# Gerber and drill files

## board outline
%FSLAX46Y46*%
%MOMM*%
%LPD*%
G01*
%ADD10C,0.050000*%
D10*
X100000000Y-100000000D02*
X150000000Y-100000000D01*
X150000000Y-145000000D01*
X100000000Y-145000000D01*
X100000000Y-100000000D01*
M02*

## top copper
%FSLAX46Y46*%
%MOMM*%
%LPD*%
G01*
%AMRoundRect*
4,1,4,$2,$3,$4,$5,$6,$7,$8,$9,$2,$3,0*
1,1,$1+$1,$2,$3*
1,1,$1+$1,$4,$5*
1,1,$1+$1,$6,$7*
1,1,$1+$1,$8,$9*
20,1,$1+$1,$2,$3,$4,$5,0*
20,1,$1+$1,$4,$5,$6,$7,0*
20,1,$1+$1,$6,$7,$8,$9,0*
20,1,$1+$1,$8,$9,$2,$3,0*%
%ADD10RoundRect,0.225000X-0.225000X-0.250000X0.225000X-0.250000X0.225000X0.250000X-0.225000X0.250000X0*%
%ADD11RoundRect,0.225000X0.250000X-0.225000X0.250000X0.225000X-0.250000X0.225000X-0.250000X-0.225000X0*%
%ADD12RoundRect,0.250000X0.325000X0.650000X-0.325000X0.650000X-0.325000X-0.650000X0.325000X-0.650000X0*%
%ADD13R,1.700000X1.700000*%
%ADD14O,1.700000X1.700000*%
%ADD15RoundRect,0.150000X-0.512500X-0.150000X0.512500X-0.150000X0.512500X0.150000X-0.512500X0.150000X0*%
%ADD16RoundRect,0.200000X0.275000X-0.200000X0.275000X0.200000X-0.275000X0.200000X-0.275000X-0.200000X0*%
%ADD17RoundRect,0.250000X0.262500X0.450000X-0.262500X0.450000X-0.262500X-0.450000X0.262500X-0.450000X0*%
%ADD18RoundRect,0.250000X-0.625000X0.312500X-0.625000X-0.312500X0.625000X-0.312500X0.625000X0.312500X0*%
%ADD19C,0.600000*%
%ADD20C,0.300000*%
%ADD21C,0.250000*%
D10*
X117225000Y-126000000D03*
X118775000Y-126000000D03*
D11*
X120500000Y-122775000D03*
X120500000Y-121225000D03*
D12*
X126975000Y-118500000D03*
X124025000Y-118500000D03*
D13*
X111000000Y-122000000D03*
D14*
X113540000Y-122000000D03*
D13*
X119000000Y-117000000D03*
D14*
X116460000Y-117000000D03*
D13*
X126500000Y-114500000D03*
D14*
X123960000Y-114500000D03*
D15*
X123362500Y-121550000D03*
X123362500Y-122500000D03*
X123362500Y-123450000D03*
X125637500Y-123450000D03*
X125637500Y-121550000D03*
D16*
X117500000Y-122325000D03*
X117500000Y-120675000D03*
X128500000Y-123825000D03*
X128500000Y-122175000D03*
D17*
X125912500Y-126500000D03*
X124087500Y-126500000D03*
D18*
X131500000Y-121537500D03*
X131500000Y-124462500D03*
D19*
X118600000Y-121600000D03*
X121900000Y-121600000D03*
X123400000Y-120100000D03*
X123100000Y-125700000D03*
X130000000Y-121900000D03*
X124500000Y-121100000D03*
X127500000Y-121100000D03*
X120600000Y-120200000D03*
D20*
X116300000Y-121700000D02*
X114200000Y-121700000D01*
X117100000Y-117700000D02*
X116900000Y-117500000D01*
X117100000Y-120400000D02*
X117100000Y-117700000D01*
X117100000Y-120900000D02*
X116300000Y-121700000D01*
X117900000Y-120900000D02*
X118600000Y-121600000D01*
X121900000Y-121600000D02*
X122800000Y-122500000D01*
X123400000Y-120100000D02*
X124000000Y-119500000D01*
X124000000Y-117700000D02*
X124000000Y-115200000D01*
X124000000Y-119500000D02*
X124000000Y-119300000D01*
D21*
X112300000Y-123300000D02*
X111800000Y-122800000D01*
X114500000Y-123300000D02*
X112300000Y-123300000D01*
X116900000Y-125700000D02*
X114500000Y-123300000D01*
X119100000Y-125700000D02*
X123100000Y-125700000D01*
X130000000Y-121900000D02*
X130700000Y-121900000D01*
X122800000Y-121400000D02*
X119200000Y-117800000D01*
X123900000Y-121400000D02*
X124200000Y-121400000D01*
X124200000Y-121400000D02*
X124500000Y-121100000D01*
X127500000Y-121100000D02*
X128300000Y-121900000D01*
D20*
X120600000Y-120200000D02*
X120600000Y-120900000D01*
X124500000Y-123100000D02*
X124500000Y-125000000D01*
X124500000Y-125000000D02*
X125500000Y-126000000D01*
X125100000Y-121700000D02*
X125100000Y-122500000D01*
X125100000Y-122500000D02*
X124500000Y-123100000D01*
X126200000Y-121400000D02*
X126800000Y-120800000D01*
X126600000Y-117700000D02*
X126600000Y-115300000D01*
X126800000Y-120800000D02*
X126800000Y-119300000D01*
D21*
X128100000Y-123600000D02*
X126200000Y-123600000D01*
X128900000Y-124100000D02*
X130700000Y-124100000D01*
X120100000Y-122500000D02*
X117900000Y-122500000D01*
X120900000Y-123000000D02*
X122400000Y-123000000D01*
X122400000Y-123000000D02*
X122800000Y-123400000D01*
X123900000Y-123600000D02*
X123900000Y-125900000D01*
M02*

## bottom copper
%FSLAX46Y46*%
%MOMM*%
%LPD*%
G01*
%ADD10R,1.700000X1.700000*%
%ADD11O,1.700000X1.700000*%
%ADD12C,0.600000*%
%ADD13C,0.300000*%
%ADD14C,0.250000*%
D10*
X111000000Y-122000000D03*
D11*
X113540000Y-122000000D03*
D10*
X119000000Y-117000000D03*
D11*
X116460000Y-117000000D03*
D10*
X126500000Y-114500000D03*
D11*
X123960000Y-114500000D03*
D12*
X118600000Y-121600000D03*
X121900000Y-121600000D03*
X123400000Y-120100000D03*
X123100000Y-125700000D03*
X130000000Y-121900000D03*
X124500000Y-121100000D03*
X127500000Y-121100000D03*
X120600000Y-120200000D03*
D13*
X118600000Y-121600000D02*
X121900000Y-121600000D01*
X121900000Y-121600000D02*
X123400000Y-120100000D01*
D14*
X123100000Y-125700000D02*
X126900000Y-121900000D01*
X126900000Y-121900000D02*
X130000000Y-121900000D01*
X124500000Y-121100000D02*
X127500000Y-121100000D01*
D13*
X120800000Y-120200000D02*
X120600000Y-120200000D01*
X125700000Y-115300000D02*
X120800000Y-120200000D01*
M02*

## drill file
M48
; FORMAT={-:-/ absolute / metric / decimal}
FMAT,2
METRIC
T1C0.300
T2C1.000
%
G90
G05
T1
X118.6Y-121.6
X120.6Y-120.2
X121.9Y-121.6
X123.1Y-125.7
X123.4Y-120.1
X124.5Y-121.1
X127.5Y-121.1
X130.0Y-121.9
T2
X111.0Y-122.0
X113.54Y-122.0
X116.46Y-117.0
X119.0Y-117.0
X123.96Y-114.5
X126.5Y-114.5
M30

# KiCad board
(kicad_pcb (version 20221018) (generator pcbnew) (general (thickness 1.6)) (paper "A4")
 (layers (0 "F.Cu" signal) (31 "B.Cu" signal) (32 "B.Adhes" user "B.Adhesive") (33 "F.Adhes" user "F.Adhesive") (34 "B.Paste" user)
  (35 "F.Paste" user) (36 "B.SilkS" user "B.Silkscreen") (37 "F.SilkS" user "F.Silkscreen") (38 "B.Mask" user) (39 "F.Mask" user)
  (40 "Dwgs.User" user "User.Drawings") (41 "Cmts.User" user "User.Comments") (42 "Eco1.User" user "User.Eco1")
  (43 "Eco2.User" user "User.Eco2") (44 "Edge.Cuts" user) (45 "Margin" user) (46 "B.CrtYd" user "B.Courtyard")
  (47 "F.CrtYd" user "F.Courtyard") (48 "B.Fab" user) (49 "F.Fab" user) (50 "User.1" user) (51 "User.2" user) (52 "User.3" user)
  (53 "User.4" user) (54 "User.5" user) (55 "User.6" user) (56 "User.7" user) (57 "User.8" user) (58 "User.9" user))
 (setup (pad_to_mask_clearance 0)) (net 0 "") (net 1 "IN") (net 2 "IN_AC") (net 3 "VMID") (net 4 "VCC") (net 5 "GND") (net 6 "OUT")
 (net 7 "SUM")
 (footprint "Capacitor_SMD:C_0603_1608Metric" (layer "F.Cu") (at 118 126)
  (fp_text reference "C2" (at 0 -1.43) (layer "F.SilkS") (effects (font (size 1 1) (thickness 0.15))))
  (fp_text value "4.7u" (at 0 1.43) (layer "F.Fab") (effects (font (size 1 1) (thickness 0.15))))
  (pad "1" smd roundrect (at -0.775 0) (size 0.9 0.95) (layers "F.Cu" "F.Paste" "F.Mask") (roundrect_rratio 0.25) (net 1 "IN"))
  (pad "2" smd roundrect (at 0.775 0) (size 0.9 0.95) (layers "F.Cu" "F.Paste" "F.Mask") (roundrect_rratio 0.25) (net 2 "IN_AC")))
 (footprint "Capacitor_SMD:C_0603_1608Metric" (layer "F.Cu") (at 120.5 122 90)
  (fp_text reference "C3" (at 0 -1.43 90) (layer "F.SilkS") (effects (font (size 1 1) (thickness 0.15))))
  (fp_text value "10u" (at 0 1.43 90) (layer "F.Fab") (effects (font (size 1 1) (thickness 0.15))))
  (pad "1" smd roundrect (at -0.775 0 90) (size 0.9 0.95) (layers "F.Cu" "F.Paste" "F.Mask") (roundrect_rratio 0.25) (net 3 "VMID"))
  (pad "2" smd roundrect (at 0.775 0 90) (size 0.9 0.95) (layers "F.Cu" "F.Paste" "F.Mask") (roundrect_rratio 0.25) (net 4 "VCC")))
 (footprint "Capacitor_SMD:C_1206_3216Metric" (layer "F.Cu") (at 125.5 118.5 180)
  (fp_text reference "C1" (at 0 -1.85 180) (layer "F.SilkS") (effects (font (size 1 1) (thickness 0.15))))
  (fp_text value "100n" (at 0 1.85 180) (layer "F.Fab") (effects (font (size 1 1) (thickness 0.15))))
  (pad "1" smd roundrect (at -1.475 0 180) (size 1.15 1.8) (layers "F.Cu" "F.Paste" "F.Mask") (roundrect_rratio 0.217391) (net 4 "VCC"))
  (pad "2" smd roundrect (at 1.475 0 180) (size 1.15 1.8) (layers "F.Cu" "F.Paste" "F.Mask") (roundrect_rratio 0.217391) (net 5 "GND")))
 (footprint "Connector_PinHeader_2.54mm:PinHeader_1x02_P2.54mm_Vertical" (layer "F.Cu") (at 111 122 90)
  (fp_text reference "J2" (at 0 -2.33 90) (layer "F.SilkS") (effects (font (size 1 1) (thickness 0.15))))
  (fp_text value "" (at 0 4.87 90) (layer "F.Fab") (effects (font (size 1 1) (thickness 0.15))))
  (pad "1" thru_hole rect (at 0 0 90) (size 1.7 1.7) (drill 1) (layers "*.Cu" "*.Mask") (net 1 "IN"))
  (pad "2" thru_hole oval (at 0 2.54 90) (size 1.7 1.7) (drill 1) (layers "*.Cu" "*.Mask") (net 5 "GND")))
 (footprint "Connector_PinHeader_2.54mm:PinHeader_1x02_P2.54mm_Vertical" (layer "F.Cu") (at 119 117 -90)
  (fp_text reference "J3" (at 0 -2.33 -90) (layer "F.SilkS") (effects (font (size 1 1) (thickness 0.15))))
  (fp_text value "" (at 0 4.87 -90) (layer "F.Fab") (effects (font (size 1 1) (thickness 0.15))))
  (pad "1" thru_hole rect (at 0 0 270) (size 1.7 1.7) (drill 1) (layers "*.Cu" "*.Mask") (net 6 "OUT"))
  (pad "2" thru_hole oval (at 0 2.54 270) (size 1.7 1.7) (drill 1) (layers "*.Cu" "*.Mask") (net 5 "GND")))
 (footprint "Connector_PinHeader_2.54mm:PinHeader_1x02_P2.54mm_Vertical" (layer "F.Cu") (at 126.5 114.5 -90)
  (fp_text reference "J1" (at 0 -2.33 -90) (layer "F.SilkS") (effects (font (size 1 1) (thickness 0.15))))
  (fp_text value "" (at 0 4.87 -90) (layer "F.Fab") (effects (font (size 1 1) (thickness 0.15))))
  (pad "1" thru_hole rect (at 0 0 270) (size 1.7 1.7) (drill 1) (layers "*.Cu" "*.Mask") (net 4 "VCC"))
  (pad "2" thru_hole oval (at 0 2.54 270) (size 1.7 1.7) (drill 1) (layers "*.Cu" "*.Mask") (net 5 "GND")))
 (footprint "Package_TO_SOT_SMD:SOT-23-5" (layer "F.Cu") (at 124.5 122.5)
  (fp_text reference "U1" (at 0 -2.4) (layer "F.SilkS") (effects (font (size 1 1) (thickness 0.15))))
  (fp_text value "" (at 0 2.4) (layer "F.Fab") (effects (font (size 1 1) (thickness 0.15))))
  (pad "1" smd roundrect (at -1.1375 -0.95) (size 1.325 0.6) (layers "F.Cu" "F.Paste" "F.Mask") (roundrect_rratio 0.25) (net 6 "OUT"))
  (pad "2" smd roundrect (at -1.1375 0) (size 1.325 0.6) (layers "F.Cu" "F.Paste" "F.Mask") (roundrect_rratio 0.25) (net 5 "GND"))
  (pad "3" smd roundrect (at -1.1375 0.95) (size 1.325 0.6) (layers "F.Cu" "F.Paste" "F.Mask") (roundrect_rratio 0.25) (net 3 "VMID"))
  (pad "4" smd roundrect (at 1.1375 0.95) (size 1.325 0.6) (layers "F.Cu" "F.Paste" "F.Mask") (roundrect_rratio 0.25) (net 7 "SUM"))
  (pad "5" smd roundrect (at 1.1375 -0.95) (size 1.325 0.6) (layers "F.Cu" "F.Paste" "F.Mask") (roundrect_rratio 0.25) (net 4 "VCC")))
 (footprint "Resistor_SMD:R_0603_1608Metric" (layer "F.Cu") (at 117.5 121.5 90)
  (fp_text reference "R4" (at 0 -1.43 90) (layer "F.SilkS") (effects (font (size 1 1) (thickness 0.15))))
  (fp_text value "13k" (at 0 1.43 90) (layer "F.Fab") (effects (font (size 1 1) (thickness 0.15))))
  (pad "1" smd roundrect (at -0.825 0 90) (size 0.8 0.95) (layers "F.Cu" "F.Paste" "F.Mask") (roundrect_rratio 0.25) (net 3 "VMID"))
  (pad "2" smd roundrect (at 0.825 0 90) (size 0.8 0.95) (layers "F.Cu" "F.Paste" "F.Mask") (roundrect_rratio 0.25) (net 5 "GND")))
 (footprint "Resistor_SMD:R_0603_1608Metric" (layer "F.Cu") (at 128.5 123 90)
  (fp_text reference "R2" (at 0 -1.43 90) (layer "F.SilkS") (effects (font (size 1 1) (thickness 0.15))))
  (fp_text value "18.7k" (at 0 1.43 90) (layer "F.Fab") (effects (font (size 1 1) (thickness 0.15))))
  (pad "1" smd roundrect (at -0.825 0 90) (size 0.8 0.95) (layers "F.Cu" "F.Paste" "F.Mask") (roundrect_rratio 0.25) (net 7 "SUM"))
  (pad "2" smd roundrect (at 0.825 0 90) (size 0.8 0.95) (layers "F.Cu" "F.Paste" "F.Mask") (roundrect_rratio 0.25) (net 6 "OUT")))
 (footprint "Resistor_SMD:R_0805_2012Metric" (layer "F.Cu") (at 125 126.5 180)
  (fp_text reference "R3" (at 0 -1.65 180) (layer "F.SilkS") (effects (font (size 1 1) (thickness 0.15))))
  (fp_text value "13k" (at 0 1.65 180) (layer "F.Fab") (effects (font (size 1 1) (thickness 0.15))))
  (pad "1" smd roundrect (at -0.9125 0 180) (size 1.025 1.4) (layers "F.Cu" "F.Paste" "F.Mask") (roundrect_rratio 0.243902) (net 4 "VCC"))
  (pad "2" smd roundrect (at 0.9125 0 180) (size 1.025 1.4) (layers "F.Cu" "F.Paste" "F.Mask") (roundrect_rratio 0.243902) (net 3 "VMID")))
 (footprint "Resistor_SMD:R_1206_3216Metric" (layer "F.Cu") (at 131.5 123 -90)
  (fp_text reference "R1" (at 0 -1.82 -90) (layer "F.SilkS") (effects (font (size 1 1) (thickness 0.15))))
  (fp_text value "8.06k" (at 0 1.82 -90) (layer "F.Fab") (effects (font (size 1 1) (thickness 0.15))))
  (pad "1" smd roundrect (at -1.4625 0 270) (size 1.125 1.75) (layers "F.Cu" "F.Paste" "F.Mask") (roundrect_rratio 0.222222) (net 2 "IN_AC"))
  (pad "2" smd roundrect (at 1.4625 0 270) (size 1.125 1.75) (layers "F.Cu" "F.Paste" "F.Mask") (roundrect_rratio 0.222222) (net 7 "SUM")))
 (gr_rect (start 100 100) (end 150 145) (stroke (width 0.05) (type default)) (fill none) (layer "Edge.Cuts"))
 (segment (start 116.3 121.7) (end 114.2 121.7) (width 0.3) (layer "F.Cu") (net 5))
 (segment (start 117.1 117.7) (end 116.9 117.5) (width 0.3) (layer "F.Cu") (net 5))
 (segment (start 117.1 120.4) (end 117.1 117.7) (width 0.3) (layer "F.Cu") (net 5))
 (segment (start 117.1 120.9) (end 116.3 121.7) (width 0.3) (layer "F.Cu") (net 5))
 (segment (start 117.9 120.9) (end 118.6 121.6) (width 0.3) (layer "F.Cu") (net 5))
 (segment (start 121.9 121.6) (end 122.8 122.5) (width 0.3) (layer "F.Cu") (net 5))
 (segment (start 123.4 120.1) (end 124 119.5) (width 0.3) (layer "F.Cu") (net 5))
 (segment (start 124 117.7) (end 124 115.2) (width 0.3) (layer "F.Cu") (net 5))
 (segment (start 124 119.5) (end 124 119.3) (width 0.3) (layer "F.Cu") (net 5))
 (via (at 118.6 121.6) (size 0.6) (drill 0.3) (layers "F.Cu" "B.Cu") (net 5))
 (via (at 121.9 121.6) (size 0.6) (drill 0.3) (layers "F.Cu" "B.Cu") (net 5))
 (via (at 123.4 120.1) (size 0.6) (drill 0.3) (layers "F.Cu" "B.Cu") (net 5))
 (segment (start 112.3 123.3) (end 111.8 122.8) (width 0.25) (layer "F.Cu") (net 1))
 (segment (start 114.5 123.3) (end 112.3 123.3) (width 0.25) (layer "F.Cu") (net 1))
 (segment (start 116.9 125.7) (end 114.5 123.3) (width 0.25) (layer "F.Cu") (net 1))
 (segment (start 118.6 121.6) (end 121.9 121.6) (width 0.3) (layer "B.Cu") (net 5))
 (segment (start 119.1 125.7) (end 123.1 125.7) (width 0.25) (layer "F.Cu") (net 2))
 (segment (start 121.9 121.6) (end 123.4 120.1) (width 0.3) (layer "B.Cu") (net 5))
 (segment (start 130 121.9) (end 130.7 121.9) (width 0.25) (layer "F.Cu") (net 2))
 (via (at 123.1 125.7) (size 0.6) (drill 0.3) (layers "F.Cu" "B.Cu") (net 2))
 (via (at 130 121.9) (size 0.6) (drill 0.3) (layers "F.Cu" "B.Cu") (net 2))
 (segment (start 122.8 121.4) (end 119.2 117.8) (width 0.25) (layer "F.Cu") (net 6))
 (segment (start 123.1 125.7) (end 126.9 121.9) (width 0.25) (layer "B.Cu") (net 2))
 (segment (start 123.9 121.4) (end 124.2 121.4) (width 0.25) (layer "F.Cu") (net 6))
 (segment (start 124.2 121.4) (end 124.5 121.1) (width 0.25) (layer "F.Cu") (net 6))
 (segment (start 126.9 121.9) (end 130 121.9) (width 0.25) (layer "B.Cu") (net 2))
 (segment (start 127.5 121.1) (end 128.3 121.9) (width 0.25) (layer "F.Cu") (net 6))
 (via (at 124.5 121.1) (size 0.6) (drill 0.3) (layers "F.Cu" "B.Cu") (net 6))
 (via (at 127.5 121.1) (size 0.6) (drill 0.3) (layers "F.Cu" "B.Cu") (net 6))
 (segment (start 120.6 120.2) (end 120.6 120.9) (width 0.3) (layer "F.Cu") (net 4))
 (segment (start 124.5 121.1) (end 127.5 121.1) (width 0.25) (layer "B.Cu") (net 6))
 (segment (start 124.5 123.1) (end 124.5 125) (width 0.3) (layer "F.Cu") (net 4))
 (segment (start 124.5 125) (end 125.5 126) (width 0.3) (layer "F.Cu") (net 4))
 (segment (start 125.1 121.7) (end 125.1 122.5) (width 0.3) (layer "F.Cu") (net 4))
 (segment (start 125.1 122.5) (end 124.5 123.1) (width 0.3) (layer "F.Cu") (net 4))
 (segment (start 126.2 121.4) (end 126.8 120.8) (width 0.3) (layer "F.Cu") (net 4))
 (segment (start 126.6 117.7) (end 126.6 115.3) (width 0.3) (layer "F.Cu") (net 4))
 (segment (start 126.8 120.8) (end 126.8 119.3) (width 0.3) (layer "F.Cu") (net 4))
 (segment (start 128.1 123.6) (end 126.2 123.6) (width 0.25) (layer "F.Cu") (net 7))
 (segment (start 128.9 124.1) (end 130.7 124.1) (width 0.25) (layer "F.Cu") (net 7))
 (via (at 120.6 120.2) (size 0.6) (drill 0.3) (layers "F.Cu" "B.Cu") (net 4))
 (segment (start 120.1 122.5) (end 117.9 122.5) (width 0.25) (layer "F.Cu") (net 3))
 (segment (start 120.8 120.2) (end 120.6 120.2) (width 0.3) (layer "B.Cu") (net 4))
 (segment (start 120.9 123) (end 122.4 123) (width 0.25) (layer "F.Cu") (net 3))
 (segment (start 122.4 123) (end 122.8 123.4) (width 0.25) (layer "F.Cu") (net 3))
 (segment (start 123.9 123.6) (end 123.9 125.9) (width 0.25) (layer "F.Cu") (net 3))
 (segment (start 125.7 115.3) (end 120.8 120.2) (width 0.3) (layer "B.Cu") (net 4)))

